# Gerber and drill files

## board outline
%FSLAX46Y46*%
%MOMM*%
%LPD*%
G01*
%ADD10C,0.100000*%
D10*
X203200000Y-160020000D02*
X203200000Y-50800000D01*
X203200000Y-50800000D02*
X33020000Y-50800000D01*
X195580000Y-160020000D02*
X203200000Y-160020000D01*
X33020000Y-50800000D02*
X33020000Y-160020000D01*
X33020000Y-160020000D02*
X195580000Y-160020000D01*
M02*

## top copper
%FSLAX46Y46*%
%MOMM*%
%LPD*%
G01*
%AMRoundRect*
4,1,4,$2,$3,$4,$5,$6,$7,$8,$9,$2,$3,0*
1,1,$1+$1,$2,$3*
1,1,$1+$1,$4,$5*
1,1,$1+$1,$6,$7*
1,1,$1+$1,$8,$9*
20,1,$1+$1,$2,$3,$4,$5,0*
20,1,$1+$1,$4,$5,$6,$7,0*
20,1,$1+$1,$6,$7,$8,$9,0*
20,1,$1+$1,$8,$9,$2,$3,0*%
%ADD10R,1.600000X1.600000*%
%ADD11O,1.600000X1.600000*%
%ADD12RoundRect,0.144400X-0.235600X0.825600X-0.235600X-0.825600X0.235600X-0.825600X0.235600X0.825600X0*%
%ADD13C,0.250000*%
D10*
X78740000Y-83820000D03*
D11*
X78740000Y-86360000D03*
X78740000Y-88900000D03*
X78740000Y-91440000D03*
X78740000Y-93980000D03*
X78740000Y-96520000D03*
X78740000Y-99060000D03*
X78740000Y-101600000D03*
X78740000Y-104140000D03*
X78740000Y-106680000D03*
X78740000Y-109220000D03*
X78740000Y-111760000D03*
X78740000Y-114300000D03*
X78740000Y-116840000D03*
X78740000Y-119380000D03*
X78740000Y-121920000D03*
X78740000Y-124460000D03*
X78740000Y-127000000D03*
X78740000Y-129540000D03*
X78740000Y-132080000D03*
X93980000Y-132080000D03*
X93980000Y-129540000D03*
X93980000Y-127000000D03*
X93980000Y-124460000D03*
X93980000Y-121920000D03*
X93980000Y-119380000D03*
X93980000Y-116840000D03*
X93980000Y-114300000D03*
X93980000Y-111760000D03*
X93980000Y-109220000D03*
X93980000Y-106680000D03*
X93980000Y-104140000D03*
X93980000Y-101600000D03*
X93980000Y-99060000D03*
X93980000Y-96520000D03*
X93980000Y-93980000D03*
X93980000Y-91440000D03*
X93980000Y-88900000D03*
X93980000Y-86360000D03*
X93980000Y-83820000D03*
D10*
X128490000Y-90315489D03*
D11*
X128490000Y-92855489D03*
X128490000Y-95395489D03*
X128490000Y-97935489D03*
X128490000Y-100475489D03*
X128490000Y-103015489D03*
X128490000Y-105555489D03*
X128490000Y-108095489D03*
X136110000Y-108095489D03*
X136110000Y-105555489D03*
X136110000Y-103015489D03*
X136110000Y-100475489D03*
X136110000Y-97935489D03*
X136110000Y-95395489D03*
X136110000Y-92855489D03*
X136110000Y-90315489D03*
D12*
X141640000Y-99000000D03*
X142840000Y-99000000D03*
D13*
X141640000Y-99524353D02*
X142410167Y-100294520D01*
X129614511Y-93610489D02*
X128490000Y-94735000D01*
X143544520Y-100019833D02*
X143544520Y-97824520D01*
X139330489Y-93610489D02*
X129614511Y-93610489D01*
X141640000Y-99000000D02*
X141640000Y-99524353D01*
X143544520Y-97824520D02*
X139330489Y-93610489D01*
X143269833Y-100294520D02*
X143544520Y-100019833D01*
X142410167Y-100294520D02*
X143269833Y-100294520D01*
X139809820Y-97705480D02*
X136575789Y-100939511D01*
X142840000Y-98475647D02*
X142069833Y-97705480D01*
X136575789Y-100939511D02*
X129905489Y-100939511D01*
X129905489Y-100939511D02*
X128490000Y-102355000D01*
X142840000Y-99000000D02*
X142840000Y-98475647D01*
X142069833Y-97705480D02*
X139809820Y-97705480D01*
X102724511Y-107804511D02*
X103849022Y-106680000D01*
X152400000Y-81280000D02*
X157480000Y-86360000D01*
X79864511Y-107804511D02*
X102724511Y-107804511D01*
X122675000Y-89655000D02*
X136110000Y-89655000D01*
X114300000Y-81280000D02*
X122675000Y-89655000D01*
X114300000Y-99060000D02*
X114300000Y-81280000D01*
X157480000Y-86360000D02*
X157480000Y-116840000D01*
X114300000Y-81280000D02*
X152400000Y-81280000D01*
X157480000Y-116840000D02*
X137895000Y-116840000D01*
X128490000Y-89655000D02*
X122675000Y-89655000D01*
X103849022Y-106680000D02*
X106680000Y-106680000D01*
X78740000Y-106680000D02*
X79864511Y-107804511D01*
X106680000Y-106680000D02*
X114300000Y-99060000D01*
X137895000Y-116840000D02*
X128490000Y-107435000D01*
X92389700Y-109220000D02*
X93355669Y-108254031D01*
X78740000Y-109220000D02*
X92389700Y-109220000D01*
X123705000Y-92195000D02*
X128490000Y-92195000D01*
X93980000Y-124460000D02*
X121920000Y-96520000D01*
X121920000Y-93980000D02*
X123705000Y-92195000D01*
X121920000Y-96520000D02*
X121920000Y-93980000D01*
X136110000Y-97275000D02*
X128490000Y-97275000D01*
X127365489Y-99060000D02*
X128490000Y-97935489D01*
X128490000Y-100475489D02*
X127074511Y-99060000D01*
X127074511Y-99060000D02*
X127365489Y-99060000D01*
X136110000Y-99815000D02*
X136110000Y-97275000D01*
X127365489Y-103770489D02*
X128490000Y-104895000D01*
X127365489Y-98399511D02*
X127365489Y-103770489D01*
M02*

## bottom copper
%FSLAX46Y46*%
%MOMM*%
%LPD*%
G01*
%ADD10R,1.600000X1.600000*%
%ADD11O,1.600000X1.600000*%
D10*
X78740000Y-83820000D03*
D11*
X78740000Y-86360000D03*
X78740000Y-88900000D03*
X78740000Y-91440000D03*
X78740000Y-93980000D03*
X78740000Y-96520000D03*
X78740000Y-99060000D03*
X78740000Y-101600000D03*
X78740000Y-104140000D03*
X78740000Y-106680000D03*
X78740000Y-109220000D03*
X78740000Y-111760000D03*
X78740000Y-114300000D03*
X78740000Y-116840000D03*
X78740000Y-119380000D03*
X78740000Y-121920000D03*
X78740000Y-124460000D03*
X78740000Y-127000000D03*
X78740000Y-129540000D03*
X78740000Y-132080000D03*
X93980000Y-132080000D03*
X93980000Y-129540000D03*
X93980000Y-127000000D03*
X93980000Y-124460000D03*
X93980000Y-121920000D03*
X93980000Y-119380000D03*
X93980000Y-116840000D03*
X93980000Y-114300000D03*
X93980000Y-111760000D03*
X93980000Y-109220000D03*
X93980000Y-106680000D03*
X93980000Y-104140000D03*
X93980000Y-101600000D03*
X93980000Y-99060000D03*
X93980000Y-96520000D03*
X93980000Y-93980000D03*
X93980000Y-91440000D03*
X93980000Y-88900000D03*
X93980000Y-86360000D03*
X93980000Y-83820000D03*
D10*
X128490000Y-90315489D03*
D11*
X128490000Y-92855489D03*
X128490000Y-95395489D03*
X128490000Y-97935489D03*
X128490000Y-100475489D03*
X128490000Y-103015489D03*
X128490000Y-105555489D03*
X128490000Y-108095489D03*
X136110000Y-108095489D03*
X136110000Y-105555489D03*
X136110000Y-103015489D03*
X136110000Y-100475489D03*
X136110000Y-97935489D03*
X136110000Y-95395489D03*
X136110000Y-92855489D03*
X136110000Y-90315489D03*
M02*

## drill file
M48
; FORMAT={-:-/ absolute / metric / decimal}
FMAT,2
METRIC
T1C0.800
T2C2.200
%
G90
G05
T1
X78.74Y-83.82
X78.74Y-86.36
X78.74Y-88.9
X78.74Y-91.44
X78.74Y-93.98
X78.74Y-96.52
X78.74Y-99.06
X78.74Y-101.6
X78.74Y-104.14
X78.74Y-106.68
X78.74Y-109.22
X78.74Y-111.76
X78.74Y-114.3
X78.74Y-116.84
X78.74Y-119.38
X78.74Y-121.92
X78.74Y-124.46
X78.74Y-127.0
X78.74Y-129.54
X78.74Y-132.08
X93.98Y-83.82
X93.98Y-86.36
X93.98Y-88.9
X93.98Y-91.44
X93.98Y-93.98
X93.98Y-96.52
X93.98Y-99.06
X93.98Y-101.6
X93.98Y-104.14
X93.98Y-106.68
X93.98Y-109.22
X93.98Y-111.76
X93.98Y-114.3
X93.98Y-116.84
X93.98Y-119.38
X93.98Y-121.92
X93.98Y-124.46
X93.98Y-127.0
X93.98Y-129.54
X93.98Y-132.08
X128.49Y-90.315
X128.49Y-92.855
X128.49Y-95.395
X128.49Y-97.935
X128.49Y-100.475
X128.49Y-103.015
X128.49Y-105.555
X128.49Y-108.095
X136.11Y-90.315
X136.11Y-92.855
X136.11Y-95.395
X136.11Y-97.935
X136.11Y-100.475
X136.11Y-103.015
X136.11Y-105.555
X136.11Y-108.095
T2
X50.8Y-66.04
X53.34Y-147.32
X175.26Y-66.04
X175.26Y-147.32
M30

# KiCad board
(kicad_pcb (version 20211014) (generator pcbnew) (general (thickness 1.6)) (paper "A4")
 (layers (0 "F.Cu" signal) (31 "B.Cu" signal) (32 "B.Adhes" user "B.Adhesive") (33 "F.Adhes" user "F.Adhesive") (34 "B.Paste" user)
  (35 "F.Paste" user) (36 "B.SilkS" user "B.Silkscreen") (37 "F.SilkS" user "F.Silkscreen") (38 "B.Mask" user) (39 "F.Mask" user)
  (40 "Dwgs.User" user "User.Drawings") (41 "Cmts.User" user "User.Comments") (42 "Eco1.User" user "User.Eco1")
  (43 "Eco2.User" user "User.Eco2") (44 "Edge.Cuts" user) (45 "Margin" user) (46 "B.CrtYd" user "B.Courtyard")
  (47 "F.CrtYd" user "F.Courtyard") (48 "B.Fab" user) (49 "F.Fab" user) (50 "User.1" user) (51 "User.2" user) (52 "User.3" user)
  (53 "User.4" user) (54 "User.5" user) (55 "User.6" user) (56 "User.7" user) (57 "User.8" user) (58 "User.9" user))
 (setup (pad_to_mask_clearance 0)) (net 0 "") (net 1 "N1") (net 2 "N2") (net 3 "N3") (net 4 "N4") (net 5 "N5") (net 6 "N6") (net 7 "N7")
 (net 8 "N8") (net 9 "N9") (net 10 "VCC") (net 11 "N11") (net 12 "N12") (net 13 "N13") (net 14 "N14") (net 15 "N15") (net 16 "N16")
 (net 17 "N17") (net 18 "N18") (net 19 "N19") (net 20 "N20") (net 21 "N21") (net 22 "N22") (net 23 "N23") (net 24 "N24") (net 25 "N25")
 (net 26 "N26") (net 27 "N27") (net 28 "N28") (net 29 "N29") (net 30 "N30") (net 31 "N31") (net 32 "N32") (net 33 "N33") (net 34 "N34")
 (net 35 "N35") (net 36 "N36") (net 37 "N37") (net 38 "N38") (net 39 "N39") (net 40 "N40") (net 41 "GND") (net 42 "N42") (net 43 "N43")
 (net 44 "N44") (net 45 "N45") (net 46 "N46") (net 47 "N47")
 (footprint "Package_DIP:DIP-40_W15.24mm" (layer "F.Cu") (at 78.74 83.82)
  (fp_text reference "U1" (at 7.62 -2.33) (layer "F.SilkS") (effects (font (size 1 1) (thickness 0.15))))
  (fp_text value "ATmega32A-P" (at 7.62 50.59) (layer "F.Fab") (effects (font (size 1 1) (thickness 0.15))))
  (pad "1" thru_hole rect (at 0 0) (size 1.6 1.6) (drill 0.8) (layers *.Cu *.Mask) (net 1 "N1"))
  (pad "2" thru_hole oval (at 0 2.54) (size 1.6 1.6) (drill 0.8) (layers *.Cu *.Mask) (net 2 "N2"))
  (pad "3" thru_hole oval (at 0 5.08) (size 1.6 1.6) (drill 0.8) (layers *.Cu *.Mask) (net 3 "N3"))
  (pad "4" thru_hole oval (at 0 7.62) (size 1.6 1.6) (drill 0.8) (layers *.Cu *.Mask) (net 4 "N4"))
  (pad "5" thru_hole oval (at 0 10.16) (size 1.6 1.6) (drill 0.8) (layers *.Cu *.Mask) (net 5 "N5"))
  (pad "6" thru_hole oval (at 0 12.7) (size 1.6 1.6) (drill 0.8) (layers *.Cu *.Mask) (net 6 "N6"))
  (pad "7" thru_hole oval (at 0 15.24) (size 1.6 1.6) (drill 0.8) (layers *.Cu *.Mask) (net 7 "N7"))
  (pad "8" thru_hole oval (at 0 17.78) (size 1.6 1.6) (drill 0.8) (layers *.Cu *.Mask) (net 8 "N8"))
  (pad "9" thru_hole oval (at 0 20.32) (size 1.6 1.6) (drill 0.8) (layers *.Cu *.Mask) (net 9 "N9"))
  (pad "10" thru_hole oval (at 0 22.86) (size 1.6 1.6) (drill 0.8) (layers *.Cu *.Mask) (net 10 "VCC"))
  (pad "11" thru_hole oval (at 0 25.4) (size 1.6 1.6) (drill 0.8) (layers *.Cu *.Mask) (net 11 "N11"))
  (pad "12" thru_hole oval (at 0 27.94) (size 1.6 1.6) (drill 0.8) (layers *.Cu *.Mask) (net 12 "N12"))
  (pad "13" thru_hole oval (at 0 30.48) (size 1.6 1.6) (drill 0.8) (layers *.Cu *.Mask) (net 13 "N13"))
  (pad "14" thru_hole oval (at 0 33.02) (size 1.6 1.6) (drill 0.8) (layers *.Cu *.Mask) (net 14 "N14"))
  (pad "15" thru_hole oval (at 0 35.56) (size 1.6 1.6) (drill 0.8) (layers *.Cu *.Mask) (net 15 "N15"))
  (pad "16" thru_hole oval (at 0 38.1) (size 1.6 1.6) (drill 0.8) (layers *.Cu *.Mask) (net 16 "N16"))
  (pad "17" thru_hole oval (at 0 40.64) (size 1.6 1.6) (drill 0.8) (layers *.Cu *.Mask) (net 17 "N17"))
  (pad "18" thru_hole oval (at 0 43.18) (size 1.6 1.6) (drill 0.8) (layers *.Cu *.Mask) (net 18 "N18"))
  (pad "19" thru_hole oval (at 0 45.72) (size 1.6 1.6) (drill 0.8) (layers *.Cu *.Mask) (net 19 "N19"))
  (pad "20" thru_hole oval (at 0 48.26) (size 1.6 1.6) (drill 0.8) (layers *.Cu *.Mask) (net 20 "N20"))
  (pad "21" thru_hole oval (at 15.24 48.26) (size 1.6 1.6) (drill 0.8) (layers *.Cu *.Mask) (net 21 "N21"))
  (pad "22" thru_hole oval (at 15.24 45.72) (size 1.6 1.6) (drill 0.8) (layers *.Cu *.Mask) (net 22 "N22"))
  (pad "23" thru_hole oval (at 15.24 43.18) (size 1.6 1.6) (drill 0.8) (layers *.Cu *.Mask) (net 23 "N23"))
  (pad "24" thru_hole oval (at 15.24 40.64) (size 1.6 1.6) (drill 0.8) (layers *.Cu *.Mask) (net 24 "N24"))
  (pad "25" thru_hole oval (at 15.24 38.1) (size 1.6 1.6) (drill 0.8) (layers *.Cu *.Mask) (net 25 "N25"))
  (pad "26" thru_hole oval (at 15.24 35.56) (size 1.6 1.6) (drill 0.8) (layers *.Cu *.Mask) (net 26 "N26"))
  (pad "27" thru_hole oval (at 15.24 33.02) (size 1.6 1.6) (drill 0.8) (layers *.Cu *.Mask) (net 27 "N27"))
  (pad "28" thru_hole oval (at 15.24 30.48) (size 1.6 1.6) (drill 0.8) (layers *.Cu *.Mask) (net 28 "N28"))
  (pad "29" thru_hole oval (at 15.24 27.94) (size 1.6 1.6) (drill 0.8) (layers *.Cu *.Mask) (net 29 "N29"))
  (pad "30" thru_hole oval (at 15.24 25.4) (size 1.6 1.6) (drill 0.8) (layers *.Cu *.Mask) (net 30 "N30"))
  (pad "31" thru_hole oval (at 15.24 22.86) (size 1.6 1.6) (drill 0.8) (layers *.Cu *.Mask) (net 11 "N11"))
  (pad "32" thru_hole oval (at 15.24 20.32) (size 1.6 1.6) (drill 0.8) (layers *.Cu *.Mask) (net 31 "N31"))
  (pad "33" thru_hole oval (at 15.24 17.78) (size 1.6 1.6) (drill 0.8) (layers *.Cu *.Mask) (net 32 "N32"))
  (pad "34" thru_hole oval (at 15.24 15.24) (size 1.6 1.6) (drill 0.8) (layers *.Cu *.Mask) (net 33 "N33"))
  (pad "35" thru_hole oval (at 15.24 12.7) (size 1.6 1.6) (drill 0.8) (layers *.Cu *.Mask) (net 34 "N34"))
  (pad "36" thru_hole oval (at 15.24 10.16) (size 1.6 1.6) (drill 0.8) (layers *.Cu *.Mask) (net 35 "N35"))
  (pad "37" thru_hole oval (at 15.24 7.62) (size 1.6 1.6) (drill 0.8) (layers *.Cu *.Mask) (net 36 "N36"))
  (pad "38" thru_hole oval (at 15.24 5.08) (size 1.6 1.6) (drill 0.8) (layers *.Cu *.Mask) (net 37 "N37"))
  (pad "39" thru_hole oval (at 15.24 2.54) (size 1.6 1.6) (drill 0.8) (layers *.Cu *.Mask) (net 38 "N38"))
  (pad "40" thru_hole oval (at 15.24 0) (size 1.6 1.6) (drill 0.8) (layers *.Cu *.Mask) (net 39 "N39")))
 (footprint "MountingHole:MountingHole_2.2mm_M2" (layer "F.Cu") (at 175.26 66.04)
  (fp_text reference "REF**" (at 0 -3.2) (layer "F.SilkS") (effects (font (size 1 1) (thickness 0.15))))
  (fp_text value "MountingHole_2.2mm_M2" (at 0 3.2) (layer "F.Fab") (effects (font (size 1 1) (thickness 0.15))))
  (pad "" np_thru_hole circle (at 0 0) (size 2.2 2.2) (drill 2.2) (layers *.Cu *.Mask)))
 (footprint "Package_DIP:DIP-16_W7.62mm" (layer "F.Cu") (at 128.49 90.315489)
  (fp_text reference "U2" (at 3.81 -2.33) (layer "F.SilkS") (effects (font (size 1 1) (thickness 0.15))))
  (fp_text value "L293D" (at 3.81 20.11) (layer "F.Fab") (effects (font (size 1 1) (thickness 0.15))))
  (pad "1" thru_hole rect (at 0 0) (size 1.6 1.6) (drill 0.8) (layers *.Cu *.Mask) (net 10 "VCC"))
  (pad "2" thru_hole oval (at 0 2.54) (size 1.6 1.6) (drill 0.8) (layers *.Cu *.Mask) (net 24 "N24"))
  (pad "3" thru_hole oval (at 0 5.08) (size 1.6 1.6) (drill 0.8) (layers *.Cu *.Mask) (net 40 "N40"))
  (pad "4" thru_hole oval (at 0 7.62) (size 1.6 1.6) (drill 0.8) (layers *.Cu *.Mask) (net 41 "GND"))
  (pad "5" thru_hole oval (at 0 10.16) (size 1.6 1.6) (drill 0.8) (layers *.Cu *.Mask) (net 41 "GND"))
  (pad "6" thru_hole oval (at 0 12.7) (size 1.6 1.6) (drill 0.8) (layers *.Cu *.Mask) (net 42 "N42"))
  (pad "7" thru_hole oval (at 0 15.24) (size 1.6 1.6) (drill 0.8) (layers *.Cu *.Mask) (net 41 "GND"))
  (pad "8" thru_hole oval (at 0 17.78) (size 1.6 1.6) (drill 0.8) (layers *.Cu *.Mask) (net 10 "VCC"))
  (pad "9" thru_hole oval (at 7.62 17.78) (size 1.6 1.6) (drill 0.8) (layers *.Cu *.Mask) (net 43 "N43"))
  (pad "10" thru_hole oval (at 7.62 15.24) (size 1.6 1.6) (drill 0.8) (layers *.Cu *.Mask) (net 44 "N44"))
  (pad "11" thru_hole oval (at 7.62 12.7) (size 1.6 1.6) (drill 0.8) (layers *.Cu *.Mask) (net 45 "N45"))
  (pad "12" thru_hole oval (at 7.62 10.16) (size 1.6 1.6) (drill 0.8) (layers *.Cu *.Mask) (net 41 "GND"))
  (pad "13" thru_hole oval (at 7.62 7.62) (size 1.6 1.6) (drill 0.8) (layers *.Cu *.Mask) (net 41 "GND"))
  (pad "14" thru_hole oval (at 7.62 5.08) (size 1.6 1.6) (drill 0.8) (layers *.Cu *.Mask) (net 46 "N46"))
  (pad "15" thru_hole oval (at 7.62 2.54) (size 1.6 1.6) (drill 0.8) (layers *.Cu *.Mask) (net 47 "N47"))
  (pad "16" thru_hole oval (at 7.62 0) (size 1.6 1.6) (drill 0.8) (layers *.Cu *.Mask) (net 10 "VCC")))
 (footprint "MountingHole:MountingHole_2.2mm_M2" (layer "F.Cu") (at 50.8 66.04)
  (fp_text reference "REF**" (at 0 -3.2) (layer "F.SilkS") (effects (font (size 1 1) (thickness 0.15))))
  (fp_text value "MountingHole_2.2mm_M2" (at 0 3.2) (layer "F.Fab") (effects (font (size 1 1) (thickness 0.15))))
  (pad "" np_thru_hole circle (at 0 0) (size 2.2 2.2) (drill 2.2) (layers *.Cu *.Mask)))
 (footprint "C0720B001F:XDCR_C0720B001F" (layer "F.Cu") (at 142.24 93.98)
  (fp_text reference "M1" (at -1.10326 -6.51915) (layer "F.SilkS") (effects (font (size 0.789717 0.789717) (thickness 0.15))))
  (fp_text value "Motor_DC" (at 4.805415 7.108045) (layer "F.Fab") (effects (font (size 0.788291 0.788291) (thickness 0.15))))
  (pad "1" smd roundrect locked (at -0.6 5.02 270) (size 1.94 0.76) (layers "F.Cu" "F.Paste" "F.Mask") (roundrect_rratio 0.19)
   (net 40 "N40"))
  (pad "2" smd roundrect locked (at 0.6 5.02 270) (size 1.94 0.76) (layers "F.Cu" "F.Paste" "F.Mask") (roundrect_rratio 0.19) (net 42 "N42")))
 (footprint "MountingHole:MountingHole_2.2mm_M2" (layer "F.Cu") (at 175.26 147.32)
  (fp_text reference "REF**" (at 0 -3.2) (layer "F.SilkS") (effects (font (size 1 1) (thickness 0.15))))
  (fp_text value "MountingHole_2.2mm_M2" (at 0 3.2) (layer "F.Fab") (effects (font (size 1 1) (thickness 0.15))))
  (pad "" np_thru_hole circle (at 0 0) (size 2.2 2.2) (drill 2.2) (layers *.Cu *.Mask)))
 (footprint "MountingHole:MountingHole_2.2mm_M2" (layer "F.Cu") (at 53.34 147.32)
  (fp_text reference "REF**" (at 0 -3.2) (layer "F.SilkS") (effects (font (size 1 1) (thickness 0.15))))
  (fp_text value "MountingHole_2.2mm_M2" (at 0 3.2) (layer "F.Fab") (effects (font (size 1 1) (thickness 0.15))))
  (pad "" np_thru_hole circle (at 0 0) (size 2.2 2.2) (drill 2.2) (layers *.Cu *.Mask)))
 (gr_line (start 203.2 160.02) (end 203.2 50.8) (layer "Edge.Cuts") (width 0.1))
 (gr_line (start 203.2 50.8) (end 33.02 50.8) (layer "Edge.Cuts") (width 0.1))
 (gr_line (start 195.58 160.02) (end 203.2 160.02) (layer "Edge.Cuts") (width 0.1))
 (gr_line (start 33.02 50.8) (end 33.02 160.02) (layer "Edge.Cuts") (width 0.1))
 (gr_line (start 33.02 160.02) (end 195.58 160.02) (layer "Edge.Cuts") (width 0.1))
 (segment (start 141.64 99.524353) (end 142.410167 100.29452) (width 0.25) (layer "F.Cu") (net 40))
 (segment (start 129.614511 93.610489) (end 128.49 94.735) (width 0.25) (layer "F.Cu") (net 40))
 (segment (start 143.54452 100.019833) (end 143.54452 97.82452) (width 0.25) (layer "F.Cu") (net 40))
 (segment (start 139.330489 93.610489) (end 129.614511 93.610489) (width 0.25) (layer "F.Cu") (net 40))
 (segment (start 141.64 99) (end 141.64 99.524353) (width 0.25) (layer "F.Cu") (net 40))
 (segment (start 143.54452 97.82452) (end 139.330489 93.610489) (width 0.25) (layer "F.Cu") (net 40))
 (segment (start 143.269833 100.29452) (end 143.54452 100.019833) (width 0.25) (layer "F.Cu") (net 40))
 (segment (start 142.410167 100.29452) (end 143.269833 100.29452) (width 0.25) (layer "F.Cu") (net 40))
 (segment (start 139.80982 97.70548) (end 136.575789 100.939511) (width 0.25) (layer "F.Cu") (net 42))
 (segment (start 142.84 98.475647) (end 142.069833 97.70548) (width 0.25) (layer "F.Cu") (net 42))
 (segment (start 136.575789 100.939511) (end 129.905489 100.939511) (width 0.25) (layer "F.Cu") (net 42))
 (segment (start 129.905489 100.939511) (end 128.49 102.355) (width 0.25) (layer "F.Cu") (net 42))
 (segment (start 142.84 99) (end 142.84 98.475647) (width 0.25) (layer "F.Cu") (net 42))
 (segment (start 142.069833 97.70548) (end 139.80982 97.70548) (width 0.25) (layer "F.Cu") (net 42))
 (segment (start 102.724511 107.804511) (end 103.849022 106.68) (width 0.25) (layer "F.Cu") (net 10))
 (segment (start 152.4 81.28) (end 157.48 86.36) (width 0.25) (layer "F.Cu") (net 10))
 (segment (start 79.864511 107.804511) (end 102.724511 107.804511) (width 0.25) (layer "F.Cu") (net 10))
 (segment (start 122.675 89.655) (end 136.11 89.655) (width 0.25) (layer "F.Cu") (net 10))
 (segment (start 114.3 81.28) (end 122.675 89.655) (width 0.25) (layer "F.Cu") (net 10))
 (segment (start 114.3 99.06) (end 114.3 81.28) (width 0.25) (layer "F.Cu") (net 10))
 (segment (start 157.48 86.36) (end 157.48 116.84) (width 0.25) (layer "F.Cu") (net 10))
 (segment (start 114.3 81.28) (end 152.4 81.28) (width 0.25) (layer "F.Cu") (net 10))
 (segment (start 157.48 116.84) (end 137.895 116.84) (width 0.25) (layer "F.Cu") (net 10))
 (segment (start 128.49 89.655) (end 122.675 89.655) (width 0.25) (layer "F.Cu") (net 10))
 (segment (start 103.849022 106.68) (end 106.68 106.68) (width 0.25) (layer "F.Cu") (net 10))
 (segment (start 78.74 106.68) (end 79.864511 107.804511) (width 0.25) (layer "F.Cu") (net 10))
 (segment (start 106.68 106.68) (end 114.3 99.06) (width 0.25) (layer "F.Cu") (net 10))
 (segment (start 137.895 116.84) (end 128.49 107.435) (width 0.25) (layer "F.Cu") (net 10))
 (segment (start 92.3897 109.22) (end 93.355669 108.254031) (width 0.25) (layer "F.Cu") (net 11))
 (segment (start 78.74 109.22) (end 92.3897 109.22) (width 0.25) (layer "F.Cu") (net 11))
 (segment (start 123.705 92.195) (end 128.49 92.195) (width 0.25) (layer "F.Cu") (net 24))
 (segment (start 93.98 124.46) (end 121.92 96.52) (width 0.25) (layer "F.Cu") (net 24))
 (segment (start 121.92 93.98) (end 123.705 92.195) (width 0.25) (layer "F.Cu") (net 24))
 (segment (start 121.92 96.52) (end 121.92 93.98) (width 0.25) (layer "F.Cu") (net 24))
 (segment (start 136.11 97.275) (end 128.49 97.275) (width 0.25) (layer "F.Cu") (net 41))
 (segment (start 127.365489 99.06) (end 128.49 97.935489) (width 0.25) (layer "F.Cu") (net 41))
 (segment (start 128.49 100.475489) (end 127.074511 99.06) (width 0.25) (layer "F.Cu") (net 41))
 (segment (start 127.074511 99.06) (end 127.365489 99.06) (width 0.25) (layer "F.Cu") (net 41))
 (segment (start 136.11 99.815) (end 136.11 97.275) (width 0.25) (layer "F.Cu") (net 41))
 (segment (start 127.365489 103.770489) (end 128.49 104.895) (width 0.25) (layer "F.Cu") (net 41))
 (segment (start 127.365489 98.399511) (end 127.365489 103.770489) (width 0.25) (layer "F.Cu") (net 41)))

